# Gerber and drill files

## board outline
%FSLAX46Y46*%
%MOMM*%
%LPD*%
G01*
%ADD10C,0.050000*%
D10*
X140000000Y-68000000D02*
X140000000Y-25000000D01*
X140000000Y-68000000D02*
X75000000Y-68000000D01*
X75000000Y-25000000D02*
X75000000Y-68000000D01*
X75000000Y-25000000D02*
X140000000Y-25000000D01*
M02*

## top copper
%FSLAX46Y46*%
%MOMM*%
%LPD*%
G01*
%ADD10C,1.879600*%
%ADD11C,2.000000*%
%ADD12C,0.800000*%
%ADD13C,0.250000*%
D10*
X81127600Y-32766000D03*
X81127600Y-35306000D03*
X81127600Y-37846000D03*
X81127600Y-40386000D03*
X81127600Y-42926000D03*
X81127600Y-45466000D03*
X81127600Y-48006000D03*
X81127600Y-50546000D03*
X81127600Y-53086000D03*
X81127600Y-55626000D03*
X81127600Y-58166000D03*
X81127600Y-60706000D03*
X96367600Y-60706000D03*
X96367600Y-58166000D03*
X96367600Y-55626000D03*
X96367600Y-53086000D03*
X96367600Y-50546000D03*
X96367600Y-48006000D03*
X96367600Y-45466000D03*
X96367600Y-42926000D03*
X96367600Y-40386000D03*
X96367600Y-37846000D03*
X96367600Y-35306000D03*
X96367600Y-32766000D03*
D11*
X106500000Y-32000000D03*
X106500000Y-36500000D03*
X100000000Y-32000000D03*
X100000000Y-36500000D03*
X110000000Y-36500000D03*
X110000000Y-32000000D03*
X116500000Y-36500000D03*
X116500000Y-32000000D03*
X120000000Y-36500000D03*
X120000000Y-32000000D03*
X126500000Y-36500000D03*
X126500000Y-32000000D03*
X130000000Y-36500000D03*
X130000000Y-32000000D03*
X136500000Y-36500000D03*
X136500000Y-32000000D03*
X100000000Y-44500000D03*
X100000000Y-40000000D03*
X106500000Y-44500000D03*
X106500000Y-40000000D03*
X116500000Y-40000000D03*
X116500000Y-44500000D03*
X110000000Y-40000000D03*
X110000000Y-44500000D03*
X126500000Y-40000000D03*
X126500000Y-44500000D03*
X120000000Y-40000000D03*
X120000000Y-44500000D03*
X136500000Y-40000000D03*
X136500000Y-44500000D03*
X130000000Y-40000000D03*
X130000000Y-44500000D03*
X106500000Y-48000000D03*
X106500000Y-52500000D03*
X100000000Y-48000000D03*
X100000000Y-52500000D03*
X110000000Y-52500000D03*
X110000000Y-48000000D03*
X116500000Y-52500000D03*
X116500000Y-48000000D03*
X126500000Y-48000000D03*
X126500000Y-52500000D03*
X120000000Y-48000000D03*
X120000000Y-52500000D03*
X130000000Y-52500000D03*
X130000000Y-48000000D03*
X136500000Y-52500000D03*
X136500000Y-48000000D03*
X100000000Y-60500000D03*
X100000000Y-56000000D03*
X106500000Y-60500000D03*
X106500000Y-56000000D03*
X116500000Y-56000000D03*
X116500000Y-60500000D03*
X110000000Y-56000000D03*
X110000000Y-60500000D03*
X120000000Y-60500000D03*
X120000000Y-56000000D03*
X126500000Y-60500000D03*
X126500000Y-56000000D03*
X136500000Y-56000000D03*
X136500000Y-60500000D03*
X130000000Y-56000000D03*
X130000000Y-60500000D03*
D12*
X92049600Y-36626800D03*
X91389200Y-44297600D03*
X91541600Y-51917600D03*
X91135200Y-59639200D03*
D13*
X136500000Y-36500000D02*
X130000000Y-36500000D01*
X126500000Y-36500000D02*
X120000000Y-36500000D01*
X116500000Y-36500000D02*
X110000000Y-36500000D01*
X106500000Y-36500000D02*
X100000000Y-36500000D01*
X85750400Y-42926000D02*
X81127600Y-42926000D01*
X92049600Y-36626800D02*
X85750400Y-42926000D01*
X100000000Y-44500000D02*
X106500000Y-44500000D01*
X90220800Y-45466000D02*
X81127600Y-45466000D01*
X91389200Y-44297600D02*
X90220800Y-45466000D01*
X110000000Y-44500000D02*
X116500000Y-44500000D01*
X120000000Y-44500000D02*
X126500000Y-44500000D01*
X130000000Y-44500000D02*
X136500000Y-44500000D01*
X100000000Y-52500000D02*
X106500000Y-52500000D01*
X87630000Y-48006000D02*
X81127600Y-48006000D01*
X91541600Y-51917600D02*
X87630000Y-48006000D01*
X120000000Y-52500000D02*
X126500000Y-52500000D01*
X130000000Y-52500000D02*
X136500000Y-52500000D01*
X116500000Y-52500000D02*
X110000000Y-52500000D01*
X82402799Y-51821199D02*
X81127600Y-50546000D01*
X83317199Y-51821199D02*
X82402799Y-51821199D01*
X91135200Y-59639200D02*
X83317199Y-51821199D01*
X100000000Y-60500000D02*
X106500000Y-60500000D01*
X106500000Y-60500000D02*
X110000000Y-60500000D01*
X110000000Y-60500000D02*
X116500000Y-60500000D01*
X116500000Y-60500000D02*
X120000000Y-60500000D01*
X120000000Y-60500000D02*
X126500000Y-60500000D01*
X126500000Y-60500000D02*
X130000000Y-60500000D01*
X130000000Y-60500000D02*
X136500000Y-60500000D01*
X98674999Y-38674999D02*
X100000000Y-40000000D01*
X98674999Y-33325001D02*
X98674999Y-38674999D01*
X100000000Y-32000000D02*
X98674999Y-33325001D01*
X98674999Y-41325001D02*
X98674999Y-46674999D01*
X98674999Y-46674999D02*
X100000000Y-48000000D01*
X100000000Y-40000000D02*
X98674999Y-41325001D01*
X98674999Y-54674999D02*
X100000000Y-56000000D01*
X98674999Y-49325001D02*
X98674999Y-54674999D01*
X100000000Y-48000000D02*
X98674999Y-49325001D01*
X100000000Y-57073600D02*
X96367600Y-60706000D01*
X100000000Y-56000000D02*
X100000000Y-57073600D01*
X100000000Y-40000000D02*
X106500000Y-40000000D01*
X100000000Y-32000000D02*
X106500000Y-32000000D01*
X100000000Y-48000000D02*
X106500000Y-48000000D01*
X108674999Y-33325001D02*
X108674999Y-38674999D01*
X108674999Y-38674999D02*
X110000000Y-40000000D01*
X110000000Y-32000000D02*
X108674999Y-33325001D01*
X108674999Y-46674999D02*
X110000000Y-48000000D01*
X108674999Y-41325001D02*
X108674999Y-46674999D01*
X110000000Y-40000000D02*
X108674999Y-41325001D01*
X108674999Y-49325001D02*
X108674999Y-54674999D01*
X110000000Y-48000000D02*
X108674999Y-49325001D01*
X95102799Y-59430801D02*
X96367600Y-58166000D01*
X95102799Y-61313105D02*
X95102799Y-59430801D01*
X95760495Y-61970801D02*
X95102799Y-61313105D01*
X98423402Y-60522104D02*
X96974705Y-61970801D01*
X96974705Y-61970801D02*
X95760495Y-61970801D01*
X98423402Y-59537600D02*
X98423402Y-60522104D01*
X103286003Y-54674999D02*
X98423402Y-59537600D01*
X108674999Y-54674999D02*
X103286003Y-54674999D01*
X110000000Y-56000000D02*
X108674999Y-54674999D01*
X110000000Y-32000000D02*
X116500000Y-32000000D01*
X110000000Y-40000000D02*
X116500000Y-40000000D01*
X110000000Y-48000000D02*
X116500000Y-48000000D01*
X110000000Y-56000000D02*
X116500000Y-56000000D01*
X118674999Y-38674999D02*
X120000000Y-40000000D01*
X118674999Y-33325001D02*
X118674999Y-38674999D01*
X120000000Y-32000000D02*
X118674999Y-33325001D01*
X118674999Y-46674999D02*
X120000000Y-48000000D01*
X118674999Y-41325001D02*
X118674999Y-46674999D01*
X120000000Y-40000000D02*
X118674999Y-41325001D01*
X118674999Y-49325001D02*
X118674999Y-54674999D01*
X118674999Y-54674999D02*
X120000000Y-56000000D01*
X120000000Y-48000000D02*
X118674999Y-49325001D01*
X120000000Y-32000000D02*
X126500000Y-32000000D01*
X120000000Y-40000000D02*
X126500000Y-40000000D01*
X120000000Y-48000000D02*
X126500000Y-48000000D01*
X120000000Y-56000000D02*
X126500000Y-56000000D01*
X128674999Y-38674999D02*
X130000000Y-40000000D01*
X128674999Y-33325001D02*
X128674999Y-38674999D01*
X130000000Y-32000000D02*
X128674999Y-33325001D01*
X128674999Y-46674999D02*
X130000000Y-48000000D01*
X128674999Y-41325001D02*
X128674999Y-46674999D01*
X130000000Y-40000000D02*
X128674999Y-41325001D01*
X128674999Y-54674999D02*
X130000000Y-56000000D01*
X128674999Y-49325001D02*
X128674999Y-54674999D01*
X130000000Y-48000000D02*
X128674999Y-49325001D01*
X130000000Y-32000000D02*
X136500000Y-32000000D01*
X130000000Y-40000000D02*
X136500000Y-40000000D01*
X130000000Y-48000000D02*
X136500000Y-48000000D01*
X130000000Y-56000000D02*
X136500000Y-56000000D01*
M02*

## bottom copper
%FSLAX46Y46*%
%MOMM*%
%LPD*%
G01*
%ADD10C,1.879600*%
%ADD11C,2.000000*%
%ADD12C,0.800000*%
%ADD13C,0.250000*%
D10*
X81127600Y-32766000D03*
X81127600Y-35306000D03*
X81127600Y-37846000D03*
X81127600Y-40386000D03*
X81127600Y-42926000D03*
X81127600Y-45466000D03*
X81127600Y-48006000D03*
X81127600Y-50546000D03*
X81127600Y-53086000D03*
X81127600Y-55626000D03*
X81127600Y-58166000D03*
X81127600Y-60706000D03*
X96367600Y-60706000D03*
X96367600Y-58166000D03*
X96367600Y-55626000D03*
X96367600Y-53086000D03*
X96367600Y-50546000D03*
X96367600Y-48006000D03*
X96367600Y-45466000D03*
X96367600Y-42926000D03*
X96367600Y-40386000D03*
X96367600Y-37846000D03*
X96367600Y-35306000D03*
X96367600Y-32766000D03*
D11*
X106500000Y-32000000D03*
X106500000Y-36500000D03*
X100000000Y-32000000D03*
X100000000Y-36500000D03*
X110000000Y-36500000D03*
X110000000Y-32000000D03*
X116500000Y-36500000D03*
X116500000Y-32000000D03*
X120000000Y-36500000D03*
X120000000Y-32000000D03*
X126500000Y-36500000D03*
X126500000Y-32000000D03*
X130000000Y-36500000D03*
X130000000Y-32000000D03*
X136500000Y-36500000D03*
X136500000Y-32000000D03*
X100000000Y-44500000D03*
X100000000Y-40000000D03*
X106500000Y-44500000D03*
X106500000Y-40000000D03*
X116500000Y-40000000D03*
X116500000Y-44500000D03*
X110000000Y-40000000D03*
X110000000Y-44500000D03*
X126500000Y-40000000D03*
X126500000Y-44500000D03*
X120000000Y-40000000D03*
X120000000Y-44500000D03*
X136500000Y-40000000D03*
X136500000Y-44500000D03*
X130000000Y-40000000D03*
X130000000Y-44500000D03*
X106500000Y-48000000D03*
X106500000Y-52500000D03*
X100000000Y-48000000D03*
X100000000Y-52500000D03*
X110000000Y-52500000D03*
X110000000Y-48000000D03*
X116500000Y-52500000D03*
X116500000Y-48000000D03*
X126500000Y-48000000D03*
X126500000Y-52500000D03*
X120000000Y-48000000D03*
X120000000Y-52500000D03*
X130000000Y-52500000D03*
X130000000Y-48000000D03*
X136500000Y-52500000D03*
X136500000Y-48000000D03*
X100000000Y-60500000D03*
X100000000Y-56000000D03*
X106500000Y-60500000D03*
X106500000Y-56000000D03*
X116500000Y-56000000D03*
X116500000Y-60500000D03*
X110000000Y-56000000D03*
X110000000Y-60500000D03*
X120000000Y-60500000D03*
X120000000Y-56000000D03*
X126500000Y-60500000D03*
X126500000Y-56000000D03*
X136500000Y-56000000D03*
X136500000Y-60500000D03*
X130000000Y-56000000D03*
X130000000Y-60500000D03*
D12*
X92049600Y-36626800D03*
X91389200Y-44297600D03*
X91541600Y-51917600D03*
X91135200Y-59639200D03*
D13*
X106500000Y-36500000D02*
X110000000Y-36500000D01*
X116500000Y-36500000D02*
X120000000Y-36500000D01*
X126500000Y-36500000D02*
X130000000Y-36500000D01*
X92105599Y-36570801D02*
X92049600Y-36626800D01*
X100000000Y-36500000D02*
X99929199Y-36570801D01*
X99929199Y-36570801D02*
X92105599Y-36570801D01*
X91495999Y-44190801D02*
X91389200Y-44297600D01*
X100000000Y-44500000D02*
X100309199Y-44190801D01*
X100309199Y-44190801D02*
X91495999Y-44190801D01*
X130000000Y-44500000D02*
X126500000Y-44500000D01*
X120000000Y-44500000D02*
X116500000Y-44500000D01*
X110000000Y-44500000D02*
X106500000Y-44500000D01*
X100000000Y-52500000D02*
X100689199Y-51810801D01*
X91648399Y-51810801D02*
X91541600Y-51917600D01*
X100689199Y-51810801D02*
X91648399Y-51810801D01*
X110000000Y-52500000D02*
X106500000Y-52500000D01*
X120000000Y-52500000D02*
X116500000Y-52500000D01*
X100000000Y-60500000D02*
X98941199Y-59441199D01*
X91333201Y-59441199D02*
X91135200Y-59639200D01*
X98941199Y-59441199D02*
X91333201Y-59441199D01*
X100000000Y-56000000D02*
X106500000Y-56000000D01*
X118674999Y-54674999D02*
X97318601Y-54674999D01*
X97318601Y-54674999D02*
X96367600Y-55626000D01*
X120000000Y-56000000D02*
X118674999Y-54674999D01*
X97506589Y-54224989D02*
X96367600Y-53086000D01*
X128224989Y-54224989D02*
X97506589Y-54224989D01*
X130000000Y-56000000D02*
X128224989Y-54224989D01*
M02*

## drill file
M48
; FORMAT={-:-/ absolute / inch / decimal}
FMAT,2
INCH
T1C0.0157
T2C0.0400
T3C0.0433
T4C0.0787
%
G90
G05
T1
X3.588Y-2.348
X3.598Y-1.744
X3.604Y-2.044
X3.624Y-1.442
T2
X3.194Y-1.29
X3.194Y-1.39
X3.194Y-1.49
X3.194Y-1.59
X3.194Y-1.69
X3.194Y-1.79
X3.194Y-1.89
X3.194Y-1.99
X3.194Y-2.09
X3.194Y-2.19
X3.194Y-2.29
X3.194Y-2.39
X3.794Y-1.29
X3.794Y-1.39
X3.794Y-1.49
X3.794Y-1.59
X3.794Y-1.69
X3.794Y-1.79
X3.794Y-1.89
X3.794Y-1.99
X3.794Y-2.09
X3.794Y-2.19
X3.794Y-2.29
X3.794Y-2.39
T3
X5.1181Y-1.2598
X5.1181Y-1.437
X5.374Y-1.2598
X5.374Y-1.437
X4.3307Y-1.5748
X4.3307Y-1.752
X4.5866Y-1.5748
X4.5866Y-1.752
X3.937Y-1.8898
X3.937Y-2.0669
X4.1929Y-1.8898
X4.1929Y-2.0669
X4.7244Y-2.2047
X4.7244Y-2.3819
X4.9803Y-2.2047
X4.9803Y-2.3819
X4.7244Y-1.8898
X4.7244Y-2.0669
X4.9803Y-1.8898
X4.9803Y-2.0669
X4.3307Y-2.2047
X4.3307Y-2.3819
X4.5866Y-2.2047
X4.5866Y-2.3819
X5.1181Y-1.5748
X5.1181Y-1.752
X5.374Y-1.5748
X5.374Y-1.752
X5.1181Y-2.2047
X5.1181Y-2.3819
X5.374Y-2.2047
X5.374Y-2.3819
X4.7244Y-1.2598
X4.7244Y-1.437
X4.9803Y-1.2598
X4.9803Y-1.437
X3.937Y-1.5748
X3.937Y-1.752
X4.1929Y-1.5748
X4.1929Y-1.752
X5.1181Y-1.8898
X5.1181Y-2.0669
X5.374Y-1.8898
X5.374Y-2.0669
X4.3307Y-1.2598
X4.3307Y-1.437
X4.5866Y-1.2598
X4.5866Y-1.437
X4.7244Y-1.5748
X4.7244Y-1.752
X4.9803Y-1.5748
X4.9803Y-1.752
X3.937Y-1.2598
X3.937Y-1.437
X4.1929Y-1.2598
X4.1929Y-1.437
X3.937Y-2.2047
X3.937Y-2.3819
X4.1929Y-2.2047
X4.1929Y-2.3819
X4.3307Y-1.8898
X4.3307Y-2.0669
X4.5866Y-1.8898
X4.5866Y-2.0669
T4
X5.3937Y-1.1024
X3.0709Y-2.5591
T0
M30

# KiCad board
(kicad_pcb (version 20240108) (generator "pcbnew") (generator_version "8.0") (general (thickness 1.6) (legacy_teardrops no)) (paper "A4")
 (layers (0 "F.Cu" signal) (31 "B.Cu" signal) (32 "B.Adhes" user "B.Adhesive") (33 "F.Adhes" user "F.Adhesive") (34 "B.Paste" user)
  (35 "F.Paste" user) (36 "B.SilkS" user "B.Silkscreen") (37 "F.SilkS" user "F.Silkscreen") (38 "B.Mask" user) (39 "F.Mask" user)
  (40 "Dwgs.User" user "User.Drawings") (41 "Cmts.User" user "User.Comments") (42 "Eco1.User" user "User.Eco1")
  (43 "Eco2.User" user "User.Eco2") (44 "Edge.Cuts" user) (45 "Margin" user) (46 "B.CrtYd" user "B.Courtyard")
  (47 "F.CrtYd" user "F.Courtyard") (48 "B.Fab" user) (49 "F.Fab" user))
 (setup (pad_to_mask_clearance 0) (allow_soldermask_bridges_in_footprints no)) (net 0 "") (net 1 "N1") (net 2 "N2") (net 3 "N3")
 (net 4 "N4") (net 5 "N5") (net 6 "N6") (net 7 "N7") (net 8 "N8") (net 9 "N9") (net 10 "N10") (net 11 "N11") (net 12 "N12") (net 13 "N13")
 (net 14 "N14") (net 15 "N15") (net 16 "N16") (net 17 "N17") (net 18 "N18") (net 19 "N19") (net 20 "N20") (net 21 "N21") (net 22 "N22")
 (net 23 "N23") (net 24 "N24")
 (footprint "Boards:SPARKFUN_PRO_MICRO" (layer "F.Cu") (at 88.7476 45.466)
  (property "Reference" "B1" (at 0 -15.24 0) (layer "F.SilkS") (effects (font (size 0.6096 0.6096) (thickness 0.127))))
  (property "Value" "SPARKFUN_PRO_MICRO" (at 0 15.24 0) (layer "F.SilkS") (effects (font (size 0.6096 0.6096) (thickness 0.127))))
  (pad "1" thru_hole circle (at -7.62 -12.7) (size 1.8796 1.8796) (drill 1.016) (layers "*.Cu" "*.Mask") (remove_unused_layers no)
   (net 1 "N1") (solder_mask_margin 0.1016))
  (pad "2" thru_hole circle (at -7.62 -10.16) (size 1.8796 1.8796) (drill 1.016) (layers "*.Cu" "*.Mask") (remove_unused_layers no)
   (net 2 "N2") (solder_mask_margin 0.1016))
  (pad "3" thru_hole circle (at -7.62 -7.62) (size 1.8796 1.8796) (drill 1.016) (layers "*.Cu" "*.Mask") (remove_unused_layers no)
   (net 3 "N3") (solder_mask_margin 0.1016))
  (pad "4" thru_hole circle (at -7.62 -5.08) (size 1.8796 1.8796) (drill 1.016) (layers "*.Cu" "*.Mask") (remove_unused_layers no)
   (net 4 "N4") (solder_mask_margin 0.1016))
  (pad "5" thru_hole circle (at -7.62 -2.54) (size 1.8796 1.8796) (drill 1.016) (layers "*.Cu" "*.Mask") (remove_unused_layers no)
   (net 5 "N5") (solder_mask_margin 0.1016))
  (pad "6" thru_hole circle (at -7.62 0) (size 1.8796 1.8796) (drill 1.016) (layers "*.Cu" "*.Mask") (remove_unused_layers no) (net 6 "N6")
   (solder_mask_margin 0.1016))
  (pad "7" thru_hole circle (at -7.62 2.54) (size 1.8796 1.8796) (drill 1.016) (layers "*.Cu" "*.Mask") (remove_unused_layers no)
   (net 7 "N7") (solder_mask_margin 0.1016))
  (pad "8" thru_hole circle (at -7.62 5.08) (size 1.8796 1.8796) (drill 1.016) (layers "*.Cu" "*.Mask") (remove_unused_layers no)
   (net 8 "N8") (solder_mask_margin 0.1016))
  (pad "9" thru_hole circle (at -7.62 7.62) (size 1.8796 1.8796) (drill 1.016) (layers "*.Cu" "*.Mask") (remove_unused_layers no)
   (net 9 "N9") (solder_mask_margin 0.1016))
  (pad "10" thru_hole circle (at -7.62 10.16) (size 1.8796 1.8796) (drill 1.016) (layers "*.Cu" "*.Mask") (remove_unused_layers no)
   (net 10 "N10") (solder_mask_margin 0.1016))
  (pad "11" thru_hole circle (at -7.62 12.7) (size 1.8796 1.8796) (drill 1.016) (layers "*.Cu" "*.Mask") (remove_unused_layers no)
   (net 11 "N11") (solder_mask_margin 0.1016))
  (pad "12" thru_hole circle (at -7.62 15.24) (size 1.8796 1.8796) (drill 1.016) (layers "*.Cu" "*.Mask") (remove_unused_layers no)
   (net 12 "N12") (solder_mask_margin 0.1016))
  (pad "13" thru_hole circle (at 7.62 15.24) (size 1.8796 1.8796) (drill 1.016) (layers "*.Cu" "*.Mask") (remove_unused_layers no)
   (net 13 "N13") (solder_mask_margin 0.1016))
  (pad "14" thru_hole circle (at 7.62 12.7) (size 1.8796 1.8796) (drill 1.016) (layers "*.Cu" "*.Mask") (remove_unused_layers no)
   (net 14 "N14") (solder_mask_margin 0.1016))
  (pad "15" thru_hole circle (at 7.62 10.16) (size 1.8796 1.8796) (drill 1.016) (layers "*.Cu" "*.Mask") (remove_unused_layers no)
   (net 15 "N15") (solder_mask_margin 0.1016))
  (pad "16" thru_hole circle (at 7.62 7.62) (size 1.8796 1.8796) (drill 1.016) (layers "*.Cu" "*.Mask") (remove_unused_layers no)
   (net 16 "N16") (solder_mask_margin 0.1016))
  (pad "17" thru_hole circle (at 7.62 5.08) (size 1.8796 1.8796) (drill 1.016) (layers "*.Cu" "*.Mask") (remove_unused_layers no)
   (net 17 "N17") (solder_mask_margin 0.1016))
  (pad "18" thru_hole circle (at 7.62 2.54) (size 1.8796 1.8796) (drill 1.016) (layers "*.Cu" "*.Mask") (remove_unused_layers no)
   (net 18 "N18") (solder_mask_margin 0.1016))
  (pad "19" thru_hole circle (at 7.62 0) (size 1.8796 1.8796) (drill 1.016) (layers "*.Cu" "*.Mask") (remove_unused_layers no)
   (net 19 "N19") (solder_mask_margin 0.1016))
  (pad "20" thru_hole circle (at 7.62 -2.54) (size 1.8796 1.8796) (drill 1.016) (layers "*.Cu" "*.Mask") (remove_unused_layers no)
   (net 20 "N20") (solder_mask_margin 0.1016))
  (pad "21" thru_hole circle (at 7.62 -5.08) (size 1.8796 1.8796) (drill 1.016) (layers "*.Cu" "*.Mask") (remove_unused_layers no)
   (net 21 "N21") (solder_mask_margin 0.1016))
  (pad "22" thru_hole circle (at 7.62 -7.62) (size 1.8796 1.8796) (drill 1.016) (layers "*.Cu" "*.Mask") (remove_unused_layers no)
   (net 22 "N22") (solder_mask_margin 0.1016))
  (pad "23" thru_hole circle (at 7.62 -10.16) (size 1.8796 1.8796) (drill 1.016) (layers "*.Cu" "*.Mask") (remove_unused_layers no)
   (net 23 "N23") (solder_mask_margin 0.1016))
  (pad "24" thru_hole circle (at 7.62 -12.7) (size 1.8796 1.8796) (drill 1.016) (layers "*.Cu" "*.Mask") (remove_unused_layers no)
   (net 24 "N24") (solder_mask_margin 0.1016)))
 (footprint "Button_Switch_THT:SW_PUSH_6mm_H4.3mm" (layer "F.Cu") (at 100 32)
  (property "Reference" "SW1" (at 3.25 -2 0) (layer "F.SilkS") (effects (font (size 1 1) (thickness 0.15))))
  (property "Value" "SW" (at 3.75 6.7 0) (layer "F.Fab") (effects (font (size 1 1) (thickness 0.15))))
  (pad "1" thru_hole circle (at 0 0 90) (size 2 2) (drill 1.1) (layers "*.Cu" "*.Mask") (remove_unused_layers no) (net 13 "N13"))
  (pad "1" thru_hole circle (at 6.5 0 90) (size 2 2) (drill 1.1) (layers "*.Cu" "*.Mask") (remove_unused_layers no) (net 13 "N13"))
  (pad "2" thru_hole circle (at 0 4.5 90) (size 2 2) (drill 1.1) (layers "*.Cu" "*.Mask") (remove_unused_layers no) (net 5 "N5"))
  (pad "2" thru_hole circle (at 6.5 4.5 90) (size 2 2) (drill 1.1) (layers "*.Cu" "*.Mask") (remove_unused_layers no) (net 5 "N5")))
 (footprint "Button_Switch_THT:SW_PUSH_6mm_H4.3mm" (layer "F.Cu") (at 110 32)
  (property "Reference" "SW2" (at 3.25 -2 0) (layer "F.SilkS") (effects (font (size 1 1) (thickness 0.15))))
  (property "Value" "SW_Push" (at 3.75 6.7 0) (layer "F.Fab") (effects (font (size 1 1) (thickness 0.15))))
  (pad "1" thru_hole circle (at 0 0 90) (size 2 2) (drill 1.1) (layers "*.Cu" "*.Mask") (remove_unused_layers no) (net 14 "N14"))
  (pad "1" thru_hole circle (at 6.5 0 90) (size 2 2) (drill 1.1) (layers "*.Cu" "*.Mask") (remove_unused_layers no) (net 14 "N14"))
  (pad "2" thru_hole circle (at 0 4.5 90) (size 2 2) (drill 1.1) (layers "*.Cu" "*.Mask") (remove_unused_layers no) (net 5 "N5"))
  (pad "2" thru_hole circle (at 6.5 4.5 90) (size 2 2) (drill 1.1) (layers "*.Cu" "*.Mask") (remove_unused_layers no) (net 5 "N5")))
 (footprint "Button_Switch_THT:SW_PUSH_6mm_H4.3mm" (layer "F.Cu") (at 120 32)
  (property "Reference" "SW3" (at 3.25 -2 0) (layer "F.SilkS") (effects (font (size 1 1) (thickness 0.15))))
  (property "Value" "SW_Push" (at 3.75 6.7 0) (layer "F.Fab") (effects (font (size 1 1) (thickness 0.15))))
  (pad "1" thru_hole circle (at 0 0 90) (size 2 2) (drill 1.1) (layers "*.Cu" "*.Mask") (remove_unused_layers no) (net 15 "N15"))
  (pad "1" thru_hole circle (at 6.5 0 90) (size 2 2) (drill 1.1) (layers "*.Cu" "*.Mask") (remove_unused_layers no) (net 15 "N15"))
  (pad "2" thru_hole circle (at 0 4.5 90) (size 2 2) (drill 1.1) (layers "*.Cu" "*.Mask") (remove_unused_layers no) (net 5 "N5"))
  (pad "2" thru_hole circle (at 6.5 4.5 90) (size 2 2) (drill 1.1) (layers "*.Cu" "*.Mask") (remove_unused_layers no) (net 5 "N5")))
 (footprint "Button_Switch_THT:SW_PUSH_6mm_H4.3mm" (layer "F.Cu") (at 130 32)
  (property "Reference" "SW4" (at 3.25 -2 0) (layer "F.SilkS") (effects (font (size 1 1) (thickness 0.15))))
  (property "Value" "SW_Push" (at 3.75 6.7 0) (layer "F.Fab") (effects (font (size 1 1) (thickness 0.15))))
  (pad "1" thru_hole circle (at 0 0 90) (size 2 2) (drill 1.1) (layers "*.Cu" "*.Mask") (remove_unused_layers no) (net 16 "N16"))
  (pad "1" thru_hole circle (at 6.5 0 90) (size 2 2) (drill 1.1) (layers "*.Cu" "*.Mask") (remove_unused_layers no) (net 16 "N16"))
  (pad "2" thru_hole circle (at 0 4.5 90) (size 2 2) (drill 1.1) (layers "*.Cu" "*.Mask") (remove_unused_layers no) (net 5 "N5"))
  (pad "2" thru_hole circle (at 6.5 4.5 90) (size 2 2) (drill 1.1) (layers "*.Cu" "*.Mask") (remove_unused_layers no) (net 5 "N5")))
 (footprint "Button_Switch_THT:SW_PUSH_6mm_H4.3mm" (layer "F.Cu") (at 100 40)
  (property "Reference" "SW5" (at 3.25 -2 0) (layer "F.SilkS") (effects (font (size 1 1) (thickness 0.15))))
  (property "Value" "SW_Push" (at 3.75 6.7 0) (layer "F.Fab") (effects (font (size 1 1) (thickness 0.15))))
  (pad "1" thru_hole circle (at 0 0 90) (size 2 2) (drill 1.1) (layers "*.Cu" "*.Mask") (remove_unused_layers no) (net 13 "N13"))
  (pad "1" thru_hole circle (at 6.5 0 90) (size 2 2) (drill 1.1) (layers "*.Cu" "*.Mask") (remove_unused_layers no) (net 13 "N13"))
  (pad "2" thru_hole circle (at 0 4.5 90) (size 2 2) (drill 1.1) (layers "*.Cu" "*.Mask") (remove_unused_layers no) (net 6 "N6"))
  (pad "2" thru_hole circle (at 6.5 4.5 90) (size 2 2) (drill 1.1) (layers "*.Cu" "*.Mask") (remove_unused_layers no) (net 6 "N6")))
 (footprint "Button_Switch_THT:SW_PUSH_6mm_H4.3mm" (layer "F.Cu") (at 110 40)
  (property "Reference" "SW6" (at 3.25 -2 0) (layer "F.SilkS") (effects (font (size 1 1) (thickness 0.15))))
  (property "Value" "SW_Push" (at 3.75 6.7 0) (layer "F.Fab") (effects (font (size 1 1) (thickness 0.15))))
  (pad "1" thru_hole circle (at 0 0 90) (size 2 2) (drill 1.1) (layers "*.Cu" "*.Mask") (remove_unused_layers no) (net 14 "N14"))
  (pad "1" thru_hole circle (at 6.5 0 90) (size 2 2) (drill 1.1) (layers "*.Cu" "*.Mask") (remove_unused_layers no) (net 14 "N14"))
  (pad "2" thru_hole circle (at 0 4.5 90) (size 2 2) (drill 1.1) (layers "*.Cu" "*.Mask") (remove_unused_layers no) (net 6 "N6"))
  (pad "2" thru_hole circle (at 6.5 4.5 90) (size 2 2) (drill 1.1) (layers "*.Cu" "*.Mask") (remove_unused_layers no) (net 6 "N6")))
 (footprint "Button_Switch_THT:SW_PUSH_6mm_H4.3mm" (layer "F.Cu") (at 120 40)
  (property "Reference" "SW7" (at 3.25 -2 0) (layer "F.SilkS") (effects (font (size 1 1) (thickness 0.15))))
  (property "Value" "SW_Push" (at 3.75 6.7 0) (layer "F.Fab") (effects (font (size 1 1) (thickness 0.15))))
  (pad "1" thru_hole circle (at 0 0 90) (size 2 2) (drill 1.1) (layers "*.Cu" "*.Mask") (remove_unused_layers no) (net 15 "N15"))
  (pad "1" thru_hole circle (at 6.5 0 90) (size 2 2) (drill 1.1) (layers "*.Cu" "*.Mask") (remove_unused_layers no) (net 15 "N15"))
  (pad "2" thru_hole circle (at 0 4.5 90) (size 2 2) (drill 1.1) (layers "*.Cu" "*.Mask") (remove_unused_layers no) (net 6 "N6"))
  (pad "2" thru_hole circle (at 6.5 4.5 90) (size 2 2) (drill 1.1) (layers "*.Cu" "*.Mask") (remove_unused_layers no) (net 6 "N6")))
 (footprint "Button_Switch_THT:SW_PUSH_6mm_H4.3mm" (layer "F.Cu") (at 130 40)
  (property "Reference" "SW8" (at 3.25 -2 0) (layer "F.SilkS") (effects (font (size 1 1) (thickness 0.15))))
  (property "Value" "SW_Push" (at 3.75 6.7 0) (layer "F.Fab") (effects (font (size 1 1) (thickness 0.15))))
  (pad "1" thru_hole circle (at 0 0 90) (size 2 2) (drill 1.1) (layers "*.Cu" "*.Mask") (remove_unused_layers no) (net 16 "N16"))
  (pad "1" thru_hole circle (at 6.5 0 90) (size 2 2) (drill 1.1) (layers "*.Cu" "*.Mask") (remove_unused_layers no) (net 16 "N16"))
  (pad "2" thru_hole circle (at 0 4.5 90) (size 2 2) (drill 1.1) (layers "*.Cu" "*.Mask") (remove_unused_layers no) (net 6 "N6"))
  (pad "2" thru_hole circle (at 6.5 4.5 90) (size 2 2) (drill 1.1) (layers "*.Cu" "*.Mask") (remove_unused_layers no) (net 6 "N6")))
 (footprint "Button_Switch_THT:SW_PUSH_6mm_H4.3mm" (layer "F.Cu") (at 100 48)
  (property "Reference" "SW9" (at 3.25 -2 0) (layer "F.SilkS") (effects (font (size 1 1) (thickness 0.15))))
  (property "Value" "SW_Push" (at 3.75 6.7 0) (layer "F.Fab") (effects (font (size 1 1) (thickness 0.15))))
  (pad "1" thru_hole circle (at 0 0 90) (size 2 2) (drill 1.1) (layers "*.Cu" "*.Mask") (remove_unused_layers no) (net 13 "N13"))
  (pad "1" thru_hole circle (at 6.5 0 90) (size 2 2) (drill 1.1) (layers "*.Cu" "*.Mask") (remove_unused_layers no) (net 13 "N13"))
  (pad "2" thru_hole circle (at 0 4.5 90) (size 2 2) (drill 1.1) (layers "*.Cu" "*.Mask") (remove_unused_layers no) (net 7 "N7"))
  (pad "2" thru_hole circle (at 6.5 4.5 90) (size 2 2) (drill 1.1) (layers "*.Cu" "*.Mask") (remove_unused_layers no) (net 7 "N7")))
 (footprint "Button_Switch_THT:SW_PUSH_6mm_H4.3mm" (layer "F.Cu") (at 110 48)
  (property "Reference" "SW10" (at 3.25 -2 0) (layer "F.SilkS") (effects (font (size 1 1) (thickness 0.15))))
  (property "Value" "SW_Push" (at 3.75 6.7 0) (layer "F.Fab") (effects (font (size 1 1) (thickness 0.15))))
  (pad "1" thru_hole circle (at 0 0 90) (size 2 2) (drill 1.1) (layers "*.Cu" "*.Mask") (remove_unused_layers no) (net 14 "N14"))
  (pad "1" thru_hole circle (at 6.5 0 90) (size 2 2) (drill 1.1) (layers "*.Cu" "*.Mask") (remove_unused_layers no) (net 14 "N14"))
  (pad "2" thru_hole circle (at 0 4.5 90) (size 2 2) (drill 1.1) (layers "*.Cu" "*.Mask") (remove_unused_layers no) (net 7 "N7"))
  (pad "2" thru_hole circle (at 6.5 4.5 90) (size 2 2) (drill 1.1) (layers "*.Cu" "*.Mask") (remove_unused_layers no) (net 7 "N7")))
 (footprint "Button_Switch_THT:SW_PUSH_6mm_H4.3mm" (layer "F.Cu") (at 120 48)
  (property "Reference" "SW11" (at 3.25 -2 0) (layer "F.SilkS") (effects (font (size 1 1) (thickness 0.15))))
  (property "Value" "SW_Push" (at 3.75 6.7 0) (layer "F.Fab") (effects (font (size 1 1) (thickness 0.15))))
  (pad "1" thru_hole circle (at 0 0 90) (size 2 2) (drill 1.1) (layers "*.Cu" "*.Mask") (remove_unused_layers no) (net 15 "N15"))
  (pad "1" thru_hole circle (at 6.5 0 90) (size 2 2) (drill 1.1) (layers "*.Cu" "*.Mask") (remove_unused_layers no) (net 15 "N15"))
  (pad "2" thru_hole circle (at 0 4.5 90) (size 2 2) (drill 1.1) (layers "*.Cu" "*.Mask") (remove_unused_layers no) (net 7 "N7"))
  (pad "2" thru_hole circle (at 6.5 4.5 90) (size 2 2) (drill 1.1) (layers "*.Cu" "*.Mask") (remove_unused_layers no) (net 7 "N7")))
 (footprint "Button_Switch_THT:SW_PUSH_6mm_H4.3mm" (layer "F.Cu") (at 130 48)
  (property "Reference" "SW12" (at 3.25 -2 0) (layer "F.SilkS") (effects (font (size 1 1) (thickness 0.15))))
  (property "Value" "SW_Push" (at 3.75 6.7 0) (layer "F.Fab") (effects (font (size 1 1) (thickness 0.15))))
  (pad "1" thru_hole circle (at 0 0 90) (size 2 2) (drill 1.1) (layers "*.Cu" "*.Mask") (remove_unused_layers no) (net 16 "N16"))
  (pad "1" thru_hole circle (at 6.5 0 90) (size 2 2) (drill 1.1) (layers "*.Cu" "*.Mask") (remove_unused_layers no) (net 16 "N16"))
  (pad "2" thru_hole circle (at 0 4.5 90) (size 2 2) (drill 1.1) (layers "*.Cu" "*.Mask") (remove_unused_layers no) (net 7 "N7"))
  (pad "2" thru_hole circle (at 6.5 4.5 90) (size 2 2) (drill 1.1) (layers "*.Cu" "*.Mask") (remove_unused_layers no) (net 7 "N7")))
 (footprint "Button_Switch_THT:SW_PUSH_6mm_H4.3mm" (layer "F.Cu") (at 100 56)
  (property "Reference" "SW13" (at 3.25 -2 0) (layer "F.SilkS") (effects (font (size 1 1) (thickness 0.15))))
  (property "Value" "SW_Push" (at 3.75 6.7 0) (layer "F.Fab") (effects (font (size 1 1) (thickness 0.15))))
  (pad "1" thru_hole circle (at 0 0 90) (size 2 2) (drill 1.1) (layers "*.Cu" "*.Mask") (remove_unused_layers no) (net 13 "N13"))
  (pad "1" thru_hole circle (at 6.5 0 90) (size 2 2) (drill 1.1) (layers "*.Cu" "*.Mask") (remove_unused_layers no) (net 13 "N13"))
  (pad "2" thru_hole circle (at 0 4.5 90) (size 2 2) (drill 1.1) (layers "*.Cu" "*.Mask") (remove_unused_layers no) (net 8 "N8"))
  (pad "2" thru_hole circle (at 6.5 4.5 90) (size 2 2) (drill 1.1) (layers "*.Cu" "*.Mask") (remove_unused_layers no) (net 8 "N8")))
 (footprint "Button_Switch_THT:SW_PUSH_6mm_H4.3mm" (layer "F.Cu") (at 110 56)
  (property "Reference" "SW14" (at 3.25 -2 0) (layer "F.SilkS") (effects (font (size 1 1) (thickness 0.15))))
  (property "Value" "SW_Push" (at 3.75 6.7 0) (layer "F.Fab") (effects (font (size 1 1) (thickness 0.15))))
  (pad "1" thru_hole circle (at 0 0 90) (size 2 2) (drill 1.1) (layers "*.Cu" "*.Mask") (remove_unused_layers no) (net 14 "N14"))
  (pad "1" thru_hole circle (at 6.5 0 90) (size 2 2) (drill 1.1) (layers "*.Cu" "*.Mask") (remove_unused_layers no) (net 14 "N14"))
  (pad "2" thru_hole circle (at 0 4.5 90) (size 2 2) (drill 1.1) (layers "*.Cu" "*.Mask") (remove_unused_layers no) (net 8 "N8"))
  (pad "2" thru_hole circle (at 6.5 4.5 90) (size 2 2) (drill 1.1) (layers "*.Cu" "*.Mask") (remove_unused_layers no) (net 8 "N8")))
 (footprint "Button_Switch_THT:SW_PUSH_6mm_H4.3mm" (layer "F.Cu") (at 120 56)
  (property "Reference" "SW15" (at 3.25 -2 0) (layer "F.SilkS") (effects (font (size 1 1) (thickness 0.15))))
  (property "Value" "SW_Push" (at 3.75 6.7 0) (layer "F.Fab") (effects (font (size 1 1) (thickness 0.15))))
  (pad "1" thru_hole circle (at 0 0 90) (size 2 2) (drill 1.1) (layers "*.Cu" "*.Mask") (remove_unused_layers no) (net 15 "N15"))
  (pad "1" thru_hole circle (at 6.5 0 90) (size 2 2) (drill 1.1) (layers "*.Cu" "*.Mask") (remove_unused_layers no) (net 15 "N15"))
  (pad "2" thru_hole circle (at 0 4.5 90) (size 2 2) (drill 1.1) (layers "*.Cu" "*.Mask") (remove_unused_layers no) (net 8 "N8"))
  (pad "2" thru_hole circle (at 6.5 4.5 90) (size 2 2) (drill 1.1) (layers "*.Cu" "*.Mask") (remove_unused_layers no) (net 8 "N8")))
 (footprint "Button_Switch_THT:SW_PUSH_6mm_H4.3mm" (layer "F.Cu") (at 130 56)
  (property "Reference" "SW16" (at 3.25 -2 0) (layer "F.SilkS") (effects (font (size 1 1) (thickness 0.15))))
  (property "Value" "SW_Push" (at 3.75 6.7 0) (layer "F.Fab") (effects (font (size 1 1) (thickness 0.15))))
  (pad "1" thru_hole circle (at 0 0 90) (size 2 2) (drill 1.1) (layers "*.Cu" "*.Mask") (remove_unused_layers no) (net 16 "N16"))
  (pad "1" thru_hole circle (at 6.5 0 90) (size 2 2) (drill 1.1) (layers "*.Cu" "*.Mask") (remove_unused_layers no) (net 16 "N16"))
  (pad "2" thru_hole circle (at 0 4.5 90) (size 2 2) (drill 1.1) (layers "*.Cu" "*.Mask") (remove_unused_layers no) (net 8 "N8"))
  (pad "2" thru_hole circle (at 6.5 4.5 90) (size 2 2) (drill 1.1) (layers "*.Cu" "*.Mask") (remove_unused_layers no) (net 8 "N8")))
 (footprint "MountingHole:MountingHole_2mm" (layer "F.Cu") (at 137 28)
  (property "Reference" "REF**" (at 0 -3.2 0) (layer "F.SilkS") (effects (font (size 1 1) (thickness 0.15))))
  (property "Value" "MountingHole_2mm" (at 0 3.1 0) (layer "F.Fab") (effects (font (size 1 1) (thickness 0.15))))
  (pad "" np_thru_hole circle (at 0 0) (size 2 2) (drill 2) (layers "*.Cu" "*.Mask")))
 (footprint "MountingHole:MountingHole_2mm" (layer "F.Cu") (at 78 65)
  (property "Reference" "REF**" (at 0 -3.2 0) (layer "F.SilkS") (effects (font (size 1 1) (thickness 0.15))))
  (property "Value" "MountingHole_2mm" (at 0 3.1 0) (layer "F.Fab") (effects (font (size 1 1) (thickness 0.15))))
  (pad "" np_thru_hole circle (at 0 0) (size 2 2) (drill 2) (layers "*.Cu" "*.Mask")))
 (gr_line (start 140 68) (end 75 68) (stroke (width 0.05) (type solid)) (layer "Edge.Cuts"))
 (gr_line (start 140 68) (end 140 25) (stroke (width 0.05) (type solid)) (layer "Edge.Cuts"))
 (gr_line (start 75 25) (end 140 25) (stroke (width 0.05) (type solid)) (layer "Edge.Cuts"))
 (gr_line (start 75 25) (end 75 68) (stroke (width 0.05) (type solid)) (layer "Edge.Cuts"))
 (segment (start 92.0496 36.6268) (end 85.7504 42.926) (width 0.25) (layer "F.Cu") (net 5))
 (segment (start 116.5 36.5) (end 110 36.5) (width 0.25) (layer "F.Cu") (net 5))
 (segment (start 106.5 36.5) (end 100 36.5) (width 0.25) (layer "F.Cu") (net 5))
 (segment (start 85.7504 42.926) (end 81.1276 42.926) (width 0.25) (layer "F.Cu") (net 5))
 (segment (start 126.5 36.5) (end 120 36.5) (width 0.25) (layer "F.Cu") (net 5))
 (segment (start 136.5 36.5) (end 130 36.5) (width 0.25) (layer "F.Cu") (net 5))
 (via (at 92.0496 36.6268) (size 0.8) (drill 0.4) (layers "F.Cu" "B.Cu") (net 5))
 (segment (start 100 36.5) (end 99.929199 36.570801) (width 0.25) (layer "B.Cu") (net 5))
 (segment (start 106.5 36.5) (end 110 36.5) (width 0.25) (layer "B.Cu") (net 5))
 (segment (start 92.105599 36.570801) (end 92.0496 36.6268) (width 0.25) (layer "B.Cu") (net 5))
 (segment (start 116.5 36.5) (end 120 36.5) (width 0.25) (layer "B.Cu") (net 5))
 (segment (start 99.929199 36.570801) (end 92.105599 36.570801) (width 0.25) (layer "B.Cu") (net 5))
 (segment (start 126.5 36.5) (end 130 36.5) (width 0.25) (layer "B.Cu") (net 5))
 (segment (start 100 44.5) (end 106.5 44.5) (width 0.25) (layer "F.Cu") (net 6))
 (segment (start 110 44.5) (end 116.5 44.5) (width 0.25) (layer "F.Cu") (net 6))
 (segment (start 120 44.5) (end 126.5 44.5) (width 0.25) (layer "F.Cu") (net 6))
 (segment (start 91.3892 44.2976) (end 90.2208 45.466) (width 0.25) (layer "F.Cu") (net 6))
 (segment (start 90.2208 45.466) (end 81.1276 45.466) (width 0.25) (layer "F.Cu") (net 6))
 (segment (start 130 44.5) (end 136.5 44.5) (width 0.25) (layer "F.Cu") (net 6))
 (via (at 91.3892 44.2976) (size 0.8) (drill 0.4) (layers "F.Cu" "B.Cu") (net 6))
 (segment (start 100.309199 44.190801) (end 91.495999 44.190801) (width 0.25) (layer "B.Cu") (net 6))
 (segment (start 91.495999 44.190801) (end 91.3892 44.2976) (width 0.25) (layer "B.Cu") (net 6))
 (segment (start 120 44.5) (end 116.5 44.5) (width 0.25) (layer "B.Cu") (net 6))
 (segment (start 100 44.5) (end 100.309199 44.190801) (width 0.25) (layer "B.Cu") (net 6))
 (segment (start 110 44.5) (end 106.5 44.5) (width 0.25) (layer "B.Cu") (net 6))
 (segment (start 130 44.5) (end 126.5 44.5) (width 0.25) (layer "B.Cu") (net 6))
 (segment (start 87.63 48.006) (end 81.1276 48.006) (width 0.25) (layer "F.Cu") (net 7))
 (segment (start 130 52.5) (end 136.5 52.5) (width 0.25) (layer "F.Cu") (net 7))
 (segment (start 100 52.5) (end 106.5 52.5) (width 0.25) (layer "F.Cu") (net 7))
 (segment (start 91.5416 51.9176) (end 87.63 48.006) (width 0.25) (layer "F.Cu") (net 7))
 (segment (start 116.5 52.5) (end 110 52.5) (width 0.25) (layer "F.Cu") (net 7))
 (segment (start 120 52.5) (end 126.5 52.5) (width 0.25) (layer "F.Cu") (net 7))
 (via (at 91.5416 51.9176) (size 0.8) (drill 0.4) (layers "F.Cu" "B.Cu") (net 7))
 (segment (start 100 52.5) (end 100.689199 51.810801) (width 0.25) (layer "B.Cu") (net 7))
 (segment (start 100.689199 51.810801) (end 91.648399 51.810801) (width 0.25) (layer "B.Cu") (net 7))
 (segment (start 91.648399 51.810801) (end 91.5416 51.9176) (width 0.25) (layer "B.Cu") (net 7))
 (segment (start 110 52.5) (end 106.5 52.5) (width 0.25) (layer "B.Cu") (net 7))
 (segment (start 120 52.5) (end 116.5 52.5) (width 0.25) (layer "B.Cu") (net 7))
 (segment (start 100 60.5) (end 106.5 60.5) (width 0.25) (layer "F.Cu") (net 8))
 (segment (start 120 60.5) (end 126.5 60.5) (width 0.25) (layer "F.Cu") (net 8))
 (segment (start 110 60.5) (end 116.5 60.5) (width 0.25) (layer "F.Cu") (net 8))
 (segment (start 126.5 60.5) (end 130 60.5) (width 0.25) (layer "F.Cu") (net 8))
 (segment (start 91.1352 59.6392) (end 83.317199 51.821199) (width 0.25) (layer "F.Cu") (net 8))
 (segment (start 83.317199 51.821199) (end 82.402799 51.821199) (width 0.25) (layer "F.Cu") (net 8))
 (segment (start 82.402799 51.821199) (end 81.1276 50.546) (width 0.25) (layer "F.Cu") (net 8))
 (segment (start 130 60.5) (end 136.5 60.5) (width 0.25) (layer "F.Cu") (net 8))
 (segment (start 106.5 60.5) (end 110 60.5) (width 0.25) (layer "F.Cu") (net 8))
 (segment (start 116.5 60.5) (end 120 60.5) (width 0.25) (layer "F.Cu") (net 8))
 (via (at 91.1352 59.6392) (size 0.8) (drill 0.4) (layers "F.Cu" "B.Cu") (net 8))
 (segment (start 98.941199 59.441199) (end 91.333201 59.441199) (width 0.25) (layer "B.Cu") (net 8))
 (segment (start 100 60.5) (end 98.941199 59.441199) (width 0.25) (layer "B.Cu") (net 8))
 (segment (start 91.333201 59.441199) (end 91.1352 59.6392) (width 0.25) (layer "B.Cu") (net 8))
 (segment (start 100 40) (end 106.5 40) (width 0.25) (layer "F.Cu") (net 13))
 (segment (start 98.674999 41.325001) (end 98.674999 46.674999) (width 0.25) (layer "F.Cu") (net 13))
 (segment (start 100 57.0736) (end 96.3676 60.706) (width 0.25) (layer "F.Cu") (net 13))
 (segment (start 98.674999 38.674999) (end 100 40) (width 0.25) (layer "F.Cu") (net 13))
 (segment (start 100 40) (end 98.674999 41.325001) (width 0.25) (layer "F.Cu") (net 13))
 (segment (start 100 56) (end 100 57.0736) (width 0.25) (layer "F.Cu") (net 13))
 (segment (start 100 48) (end 98.674999 49.325001) (width 0.25) (layer "F.Cu") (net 13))
 (segment (start 98.674999 33.325001) (end 98.674999 38.674999) (width 0.25) (layer "F.Cu") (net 13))
 (segment (start 100 48) (end 106.5 48) (width 0.25) (layer "F.Cu") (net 13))
 (segment (start 100 32) (end 106.5 32) (width 0.25) (layer "F.Cu") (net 13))
 (segment (start 98.674999 54.674999) (end 100 56) (width 0.25) (layer "F.Cu") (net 13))
 (segment (start 98.674999 46.674999) (end 100 48) (width 0.25) (layer "F.Cu") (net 13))
 (segment (start 100 32) (end 98.674999 33.325001) (width 0.25) (layer "F.Cu") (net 13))
 (segment (start 98.674999 49.325001) (end 98.674999 54.674999) (width 0.25) (layer "F.Cu") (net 13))
 (segment (start 100 56) (end 106.5 56) (width 0.25) (layer "B.Cu") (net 13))
 (segment (start 95.102799 61.313105) (end 95.102799 59.430801) (width 0.25) (layer "F.Cu") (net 14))
 (segment (start 95.102799 59.430801) (end 96.3676 58.166) (width 0.25) (layer "F.Cu") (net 14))
 (segment (start 110 32) (end 116.5 32) (width 0.25) (layer "F.Cu") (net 14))
 (segment (start 108.674999 46.674999) (end 110 48) (width 0.25) (layer "F.Cu") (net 14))
 (segment (start 95.760495 61.970801) (end 95.102799 61.313105) (width 0.25) (layer "F.Cu") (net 14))
 (segment (start 96.974705 61.970801) (end 95.760495 61.970801) (width 0.25) (layer "F.Cu") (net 14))
 (segment (start 110 32) (end 108.674999 33.325001) (width 0.25) (layer "F.Cu") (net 14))
 (segment (start 110 40) (end 108.674999 41.325001) (width 0.25) (layer "F.Cu") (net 14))
 (segment (start 108.674999 41.325001) (end 108.674999 46.674999) (width 0.25) (layer "F.Cu") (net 14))
 (segment (start 110 48) (end 108.674999 49.325001) (width 0.25) (layer "F.Cu") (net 14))
 (segment (start 98.423402 59.5376) (end 98.423402 60.522104) (width 0.25) (layer "F.Cu") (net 14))
 (segment (start 110 48) (end 116.5 48) (width 0.25) (layer "F.Cu") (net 14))
 (segment (start 103.286003 54.674999) (end 98.423402 59.5376) (width 0.25) (layer "F.Cu") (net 14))
 (segment (start 110 56) (end 108.674999 54.674999) (width 0.25) (layer "F.Cu") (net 14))
 (segment (start 108.674999 49.325001) (end 108.674999 54.674999) (width 0.25) (layer "F.Cu") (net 14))
 (segment (start 108.674999 38.674999) (end 110 40) (width 0.25) (layer "F.Cu") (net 14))
 (segment (start 98.423402 60.522104) (end 96.974705 61.970801) (width 0.25) (layer "F.Cu") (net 14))
 (segment (start 110 40) (end 116.5 40) (width 0.25) (layer "F.Cu") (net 14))
 (segment (start 108.674999 33.325001) (end 108.674999 38.674999) (width 0.25) (layer "F.Cu") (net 14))
 (segment (start 110 56) (end 116.5 56) (width 0.25) (layer "F.Cu") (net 14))
 (segment (start 108.674999 54.674999) (end 103.286003 54.674999) (width 0.25) (layer "F.Cu") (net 14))
 (segment (start 120 32) (end 126.5 32) (width 0.25) (layer "F.Cu") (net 15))
 (segment (start 120 40) (end 126.5 40) (width 0.25) (layer "F.Cu") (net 15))
 (segment (start 118.674999 49.325001) (end 118.674999 54.674999) (width 0.25) (layer "F.Cu") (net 15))
 (segment (start 120 48) (end 126.5 48) (width 0.25) (layer "F.Cu") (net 15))
 (segment (start 120 40) (end 118.674999 41.325001) (width 0.25) (layer "F.Cu") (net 15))
 (segment (start 118.674999 41.325001) (end 118.674999 46.674999) (width 0.25) (layer "F.Cu") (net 15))
 (segment (start 118.674999 54.674999) (end 120 56) (width 0.25) (layer "F.Cu") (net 15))
 (segment (start 118.674999 46.674999) (end 120 48) (width 0.25) (layer "F.Cu") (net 15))
 (segment (start 120 56) (end 126.5 56) (width 0.25) (layer "F.Cu") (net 15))
 (segment (start 120 32) (end 118.674999 33.325001) (width 0.25) (layer "F.Cu") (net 15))
 (segment (start 120 48) (end 118.674999 49.325001) (width 0.25) (layer "F.Cu") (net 15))
 (segment (start 118.674999 38.674999) (end 120 40) (width 0.25) (layer "F.Cu") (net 15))
 (segment (start 118.674999 33.325001) (end 118.674999 38.674999) (width 0.25) (layer "F.Cu") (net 15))
 (segment (start 97.318601 54.674999) (end 96.3676 55.626) (width 0.25) (layer "B.Cu") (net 15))
 (segment (start 120 56) (end 118.674999 54.674999) (width 0.25) (layer "B.Cu") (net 15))
 (segment (start 118.674999 54.674999) (end 97.318601 54.674999) (width 0.25) (layer "B.Cu") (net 15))
 (segment (start 130 40) (end 136.5 40) (width 0.25) (layer "F.Cu") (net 16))
 (segment (start 128.674999 41.325001) (end 128.674999 46.674999) (width 0.25) (layer "F.Cu") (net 16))
 (segment (start 128.674999 33.325001) (end 128.674999 38.674999) (width 0.25) (layer "F.Cu") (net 16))
 (segment (start 128.674999 49.325001) (end 128.674999 54.674999) (width 0.25) (layer "F.Cu") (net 16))
 (segment (start 130 32) (end 128.674999 33.325001) (width 0.25) (layer "F.Cu") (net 16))
 (segment (start 128.674999 46.674999) (end 130 48) (width 0.25) (layer "F.Cu") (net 16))
 (segment (start 128.674999 54.674999) (end 130 56) (width 0.25) (layer "F.Cu") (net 16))
 (segment (start 130 56) (end 136.5 56) (width 0.25) (layer "F.Cu") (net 16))
 (segment (start 130 40) (end 128.674999 41.325001) (width 0.25) (layer "F.Cu") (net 16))
 (segment (start 128.674999 38.674999) (end 130 40) (width 0.25) (layer "F.Cu") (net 16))
 (segment (start 130 48) (end 136.5 48) (width 0.25) (layer "F.Cu") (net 16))
 (segment (start 130 48) (end 128.674999 49.325001) (width 0.25) (layer "F.Cu") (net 16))
 (segment (start 130 32) (end 136.5 32) (width 0.25) (layer "F.Cu") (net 16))
 (segment (start 130 56) (end 128.224989 54.224989) (width 0.25) (layer "B.Cu") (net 16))
 (segment (start 97.506589 54.224989) (end 96.3676 53.086) (width 0.25) (layer "B.Cu") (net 16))
 (segment (start 128.224989 54.224989) (end 97.506589 54.224989) (width 0.25) (layer "B.Cu") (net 16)))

